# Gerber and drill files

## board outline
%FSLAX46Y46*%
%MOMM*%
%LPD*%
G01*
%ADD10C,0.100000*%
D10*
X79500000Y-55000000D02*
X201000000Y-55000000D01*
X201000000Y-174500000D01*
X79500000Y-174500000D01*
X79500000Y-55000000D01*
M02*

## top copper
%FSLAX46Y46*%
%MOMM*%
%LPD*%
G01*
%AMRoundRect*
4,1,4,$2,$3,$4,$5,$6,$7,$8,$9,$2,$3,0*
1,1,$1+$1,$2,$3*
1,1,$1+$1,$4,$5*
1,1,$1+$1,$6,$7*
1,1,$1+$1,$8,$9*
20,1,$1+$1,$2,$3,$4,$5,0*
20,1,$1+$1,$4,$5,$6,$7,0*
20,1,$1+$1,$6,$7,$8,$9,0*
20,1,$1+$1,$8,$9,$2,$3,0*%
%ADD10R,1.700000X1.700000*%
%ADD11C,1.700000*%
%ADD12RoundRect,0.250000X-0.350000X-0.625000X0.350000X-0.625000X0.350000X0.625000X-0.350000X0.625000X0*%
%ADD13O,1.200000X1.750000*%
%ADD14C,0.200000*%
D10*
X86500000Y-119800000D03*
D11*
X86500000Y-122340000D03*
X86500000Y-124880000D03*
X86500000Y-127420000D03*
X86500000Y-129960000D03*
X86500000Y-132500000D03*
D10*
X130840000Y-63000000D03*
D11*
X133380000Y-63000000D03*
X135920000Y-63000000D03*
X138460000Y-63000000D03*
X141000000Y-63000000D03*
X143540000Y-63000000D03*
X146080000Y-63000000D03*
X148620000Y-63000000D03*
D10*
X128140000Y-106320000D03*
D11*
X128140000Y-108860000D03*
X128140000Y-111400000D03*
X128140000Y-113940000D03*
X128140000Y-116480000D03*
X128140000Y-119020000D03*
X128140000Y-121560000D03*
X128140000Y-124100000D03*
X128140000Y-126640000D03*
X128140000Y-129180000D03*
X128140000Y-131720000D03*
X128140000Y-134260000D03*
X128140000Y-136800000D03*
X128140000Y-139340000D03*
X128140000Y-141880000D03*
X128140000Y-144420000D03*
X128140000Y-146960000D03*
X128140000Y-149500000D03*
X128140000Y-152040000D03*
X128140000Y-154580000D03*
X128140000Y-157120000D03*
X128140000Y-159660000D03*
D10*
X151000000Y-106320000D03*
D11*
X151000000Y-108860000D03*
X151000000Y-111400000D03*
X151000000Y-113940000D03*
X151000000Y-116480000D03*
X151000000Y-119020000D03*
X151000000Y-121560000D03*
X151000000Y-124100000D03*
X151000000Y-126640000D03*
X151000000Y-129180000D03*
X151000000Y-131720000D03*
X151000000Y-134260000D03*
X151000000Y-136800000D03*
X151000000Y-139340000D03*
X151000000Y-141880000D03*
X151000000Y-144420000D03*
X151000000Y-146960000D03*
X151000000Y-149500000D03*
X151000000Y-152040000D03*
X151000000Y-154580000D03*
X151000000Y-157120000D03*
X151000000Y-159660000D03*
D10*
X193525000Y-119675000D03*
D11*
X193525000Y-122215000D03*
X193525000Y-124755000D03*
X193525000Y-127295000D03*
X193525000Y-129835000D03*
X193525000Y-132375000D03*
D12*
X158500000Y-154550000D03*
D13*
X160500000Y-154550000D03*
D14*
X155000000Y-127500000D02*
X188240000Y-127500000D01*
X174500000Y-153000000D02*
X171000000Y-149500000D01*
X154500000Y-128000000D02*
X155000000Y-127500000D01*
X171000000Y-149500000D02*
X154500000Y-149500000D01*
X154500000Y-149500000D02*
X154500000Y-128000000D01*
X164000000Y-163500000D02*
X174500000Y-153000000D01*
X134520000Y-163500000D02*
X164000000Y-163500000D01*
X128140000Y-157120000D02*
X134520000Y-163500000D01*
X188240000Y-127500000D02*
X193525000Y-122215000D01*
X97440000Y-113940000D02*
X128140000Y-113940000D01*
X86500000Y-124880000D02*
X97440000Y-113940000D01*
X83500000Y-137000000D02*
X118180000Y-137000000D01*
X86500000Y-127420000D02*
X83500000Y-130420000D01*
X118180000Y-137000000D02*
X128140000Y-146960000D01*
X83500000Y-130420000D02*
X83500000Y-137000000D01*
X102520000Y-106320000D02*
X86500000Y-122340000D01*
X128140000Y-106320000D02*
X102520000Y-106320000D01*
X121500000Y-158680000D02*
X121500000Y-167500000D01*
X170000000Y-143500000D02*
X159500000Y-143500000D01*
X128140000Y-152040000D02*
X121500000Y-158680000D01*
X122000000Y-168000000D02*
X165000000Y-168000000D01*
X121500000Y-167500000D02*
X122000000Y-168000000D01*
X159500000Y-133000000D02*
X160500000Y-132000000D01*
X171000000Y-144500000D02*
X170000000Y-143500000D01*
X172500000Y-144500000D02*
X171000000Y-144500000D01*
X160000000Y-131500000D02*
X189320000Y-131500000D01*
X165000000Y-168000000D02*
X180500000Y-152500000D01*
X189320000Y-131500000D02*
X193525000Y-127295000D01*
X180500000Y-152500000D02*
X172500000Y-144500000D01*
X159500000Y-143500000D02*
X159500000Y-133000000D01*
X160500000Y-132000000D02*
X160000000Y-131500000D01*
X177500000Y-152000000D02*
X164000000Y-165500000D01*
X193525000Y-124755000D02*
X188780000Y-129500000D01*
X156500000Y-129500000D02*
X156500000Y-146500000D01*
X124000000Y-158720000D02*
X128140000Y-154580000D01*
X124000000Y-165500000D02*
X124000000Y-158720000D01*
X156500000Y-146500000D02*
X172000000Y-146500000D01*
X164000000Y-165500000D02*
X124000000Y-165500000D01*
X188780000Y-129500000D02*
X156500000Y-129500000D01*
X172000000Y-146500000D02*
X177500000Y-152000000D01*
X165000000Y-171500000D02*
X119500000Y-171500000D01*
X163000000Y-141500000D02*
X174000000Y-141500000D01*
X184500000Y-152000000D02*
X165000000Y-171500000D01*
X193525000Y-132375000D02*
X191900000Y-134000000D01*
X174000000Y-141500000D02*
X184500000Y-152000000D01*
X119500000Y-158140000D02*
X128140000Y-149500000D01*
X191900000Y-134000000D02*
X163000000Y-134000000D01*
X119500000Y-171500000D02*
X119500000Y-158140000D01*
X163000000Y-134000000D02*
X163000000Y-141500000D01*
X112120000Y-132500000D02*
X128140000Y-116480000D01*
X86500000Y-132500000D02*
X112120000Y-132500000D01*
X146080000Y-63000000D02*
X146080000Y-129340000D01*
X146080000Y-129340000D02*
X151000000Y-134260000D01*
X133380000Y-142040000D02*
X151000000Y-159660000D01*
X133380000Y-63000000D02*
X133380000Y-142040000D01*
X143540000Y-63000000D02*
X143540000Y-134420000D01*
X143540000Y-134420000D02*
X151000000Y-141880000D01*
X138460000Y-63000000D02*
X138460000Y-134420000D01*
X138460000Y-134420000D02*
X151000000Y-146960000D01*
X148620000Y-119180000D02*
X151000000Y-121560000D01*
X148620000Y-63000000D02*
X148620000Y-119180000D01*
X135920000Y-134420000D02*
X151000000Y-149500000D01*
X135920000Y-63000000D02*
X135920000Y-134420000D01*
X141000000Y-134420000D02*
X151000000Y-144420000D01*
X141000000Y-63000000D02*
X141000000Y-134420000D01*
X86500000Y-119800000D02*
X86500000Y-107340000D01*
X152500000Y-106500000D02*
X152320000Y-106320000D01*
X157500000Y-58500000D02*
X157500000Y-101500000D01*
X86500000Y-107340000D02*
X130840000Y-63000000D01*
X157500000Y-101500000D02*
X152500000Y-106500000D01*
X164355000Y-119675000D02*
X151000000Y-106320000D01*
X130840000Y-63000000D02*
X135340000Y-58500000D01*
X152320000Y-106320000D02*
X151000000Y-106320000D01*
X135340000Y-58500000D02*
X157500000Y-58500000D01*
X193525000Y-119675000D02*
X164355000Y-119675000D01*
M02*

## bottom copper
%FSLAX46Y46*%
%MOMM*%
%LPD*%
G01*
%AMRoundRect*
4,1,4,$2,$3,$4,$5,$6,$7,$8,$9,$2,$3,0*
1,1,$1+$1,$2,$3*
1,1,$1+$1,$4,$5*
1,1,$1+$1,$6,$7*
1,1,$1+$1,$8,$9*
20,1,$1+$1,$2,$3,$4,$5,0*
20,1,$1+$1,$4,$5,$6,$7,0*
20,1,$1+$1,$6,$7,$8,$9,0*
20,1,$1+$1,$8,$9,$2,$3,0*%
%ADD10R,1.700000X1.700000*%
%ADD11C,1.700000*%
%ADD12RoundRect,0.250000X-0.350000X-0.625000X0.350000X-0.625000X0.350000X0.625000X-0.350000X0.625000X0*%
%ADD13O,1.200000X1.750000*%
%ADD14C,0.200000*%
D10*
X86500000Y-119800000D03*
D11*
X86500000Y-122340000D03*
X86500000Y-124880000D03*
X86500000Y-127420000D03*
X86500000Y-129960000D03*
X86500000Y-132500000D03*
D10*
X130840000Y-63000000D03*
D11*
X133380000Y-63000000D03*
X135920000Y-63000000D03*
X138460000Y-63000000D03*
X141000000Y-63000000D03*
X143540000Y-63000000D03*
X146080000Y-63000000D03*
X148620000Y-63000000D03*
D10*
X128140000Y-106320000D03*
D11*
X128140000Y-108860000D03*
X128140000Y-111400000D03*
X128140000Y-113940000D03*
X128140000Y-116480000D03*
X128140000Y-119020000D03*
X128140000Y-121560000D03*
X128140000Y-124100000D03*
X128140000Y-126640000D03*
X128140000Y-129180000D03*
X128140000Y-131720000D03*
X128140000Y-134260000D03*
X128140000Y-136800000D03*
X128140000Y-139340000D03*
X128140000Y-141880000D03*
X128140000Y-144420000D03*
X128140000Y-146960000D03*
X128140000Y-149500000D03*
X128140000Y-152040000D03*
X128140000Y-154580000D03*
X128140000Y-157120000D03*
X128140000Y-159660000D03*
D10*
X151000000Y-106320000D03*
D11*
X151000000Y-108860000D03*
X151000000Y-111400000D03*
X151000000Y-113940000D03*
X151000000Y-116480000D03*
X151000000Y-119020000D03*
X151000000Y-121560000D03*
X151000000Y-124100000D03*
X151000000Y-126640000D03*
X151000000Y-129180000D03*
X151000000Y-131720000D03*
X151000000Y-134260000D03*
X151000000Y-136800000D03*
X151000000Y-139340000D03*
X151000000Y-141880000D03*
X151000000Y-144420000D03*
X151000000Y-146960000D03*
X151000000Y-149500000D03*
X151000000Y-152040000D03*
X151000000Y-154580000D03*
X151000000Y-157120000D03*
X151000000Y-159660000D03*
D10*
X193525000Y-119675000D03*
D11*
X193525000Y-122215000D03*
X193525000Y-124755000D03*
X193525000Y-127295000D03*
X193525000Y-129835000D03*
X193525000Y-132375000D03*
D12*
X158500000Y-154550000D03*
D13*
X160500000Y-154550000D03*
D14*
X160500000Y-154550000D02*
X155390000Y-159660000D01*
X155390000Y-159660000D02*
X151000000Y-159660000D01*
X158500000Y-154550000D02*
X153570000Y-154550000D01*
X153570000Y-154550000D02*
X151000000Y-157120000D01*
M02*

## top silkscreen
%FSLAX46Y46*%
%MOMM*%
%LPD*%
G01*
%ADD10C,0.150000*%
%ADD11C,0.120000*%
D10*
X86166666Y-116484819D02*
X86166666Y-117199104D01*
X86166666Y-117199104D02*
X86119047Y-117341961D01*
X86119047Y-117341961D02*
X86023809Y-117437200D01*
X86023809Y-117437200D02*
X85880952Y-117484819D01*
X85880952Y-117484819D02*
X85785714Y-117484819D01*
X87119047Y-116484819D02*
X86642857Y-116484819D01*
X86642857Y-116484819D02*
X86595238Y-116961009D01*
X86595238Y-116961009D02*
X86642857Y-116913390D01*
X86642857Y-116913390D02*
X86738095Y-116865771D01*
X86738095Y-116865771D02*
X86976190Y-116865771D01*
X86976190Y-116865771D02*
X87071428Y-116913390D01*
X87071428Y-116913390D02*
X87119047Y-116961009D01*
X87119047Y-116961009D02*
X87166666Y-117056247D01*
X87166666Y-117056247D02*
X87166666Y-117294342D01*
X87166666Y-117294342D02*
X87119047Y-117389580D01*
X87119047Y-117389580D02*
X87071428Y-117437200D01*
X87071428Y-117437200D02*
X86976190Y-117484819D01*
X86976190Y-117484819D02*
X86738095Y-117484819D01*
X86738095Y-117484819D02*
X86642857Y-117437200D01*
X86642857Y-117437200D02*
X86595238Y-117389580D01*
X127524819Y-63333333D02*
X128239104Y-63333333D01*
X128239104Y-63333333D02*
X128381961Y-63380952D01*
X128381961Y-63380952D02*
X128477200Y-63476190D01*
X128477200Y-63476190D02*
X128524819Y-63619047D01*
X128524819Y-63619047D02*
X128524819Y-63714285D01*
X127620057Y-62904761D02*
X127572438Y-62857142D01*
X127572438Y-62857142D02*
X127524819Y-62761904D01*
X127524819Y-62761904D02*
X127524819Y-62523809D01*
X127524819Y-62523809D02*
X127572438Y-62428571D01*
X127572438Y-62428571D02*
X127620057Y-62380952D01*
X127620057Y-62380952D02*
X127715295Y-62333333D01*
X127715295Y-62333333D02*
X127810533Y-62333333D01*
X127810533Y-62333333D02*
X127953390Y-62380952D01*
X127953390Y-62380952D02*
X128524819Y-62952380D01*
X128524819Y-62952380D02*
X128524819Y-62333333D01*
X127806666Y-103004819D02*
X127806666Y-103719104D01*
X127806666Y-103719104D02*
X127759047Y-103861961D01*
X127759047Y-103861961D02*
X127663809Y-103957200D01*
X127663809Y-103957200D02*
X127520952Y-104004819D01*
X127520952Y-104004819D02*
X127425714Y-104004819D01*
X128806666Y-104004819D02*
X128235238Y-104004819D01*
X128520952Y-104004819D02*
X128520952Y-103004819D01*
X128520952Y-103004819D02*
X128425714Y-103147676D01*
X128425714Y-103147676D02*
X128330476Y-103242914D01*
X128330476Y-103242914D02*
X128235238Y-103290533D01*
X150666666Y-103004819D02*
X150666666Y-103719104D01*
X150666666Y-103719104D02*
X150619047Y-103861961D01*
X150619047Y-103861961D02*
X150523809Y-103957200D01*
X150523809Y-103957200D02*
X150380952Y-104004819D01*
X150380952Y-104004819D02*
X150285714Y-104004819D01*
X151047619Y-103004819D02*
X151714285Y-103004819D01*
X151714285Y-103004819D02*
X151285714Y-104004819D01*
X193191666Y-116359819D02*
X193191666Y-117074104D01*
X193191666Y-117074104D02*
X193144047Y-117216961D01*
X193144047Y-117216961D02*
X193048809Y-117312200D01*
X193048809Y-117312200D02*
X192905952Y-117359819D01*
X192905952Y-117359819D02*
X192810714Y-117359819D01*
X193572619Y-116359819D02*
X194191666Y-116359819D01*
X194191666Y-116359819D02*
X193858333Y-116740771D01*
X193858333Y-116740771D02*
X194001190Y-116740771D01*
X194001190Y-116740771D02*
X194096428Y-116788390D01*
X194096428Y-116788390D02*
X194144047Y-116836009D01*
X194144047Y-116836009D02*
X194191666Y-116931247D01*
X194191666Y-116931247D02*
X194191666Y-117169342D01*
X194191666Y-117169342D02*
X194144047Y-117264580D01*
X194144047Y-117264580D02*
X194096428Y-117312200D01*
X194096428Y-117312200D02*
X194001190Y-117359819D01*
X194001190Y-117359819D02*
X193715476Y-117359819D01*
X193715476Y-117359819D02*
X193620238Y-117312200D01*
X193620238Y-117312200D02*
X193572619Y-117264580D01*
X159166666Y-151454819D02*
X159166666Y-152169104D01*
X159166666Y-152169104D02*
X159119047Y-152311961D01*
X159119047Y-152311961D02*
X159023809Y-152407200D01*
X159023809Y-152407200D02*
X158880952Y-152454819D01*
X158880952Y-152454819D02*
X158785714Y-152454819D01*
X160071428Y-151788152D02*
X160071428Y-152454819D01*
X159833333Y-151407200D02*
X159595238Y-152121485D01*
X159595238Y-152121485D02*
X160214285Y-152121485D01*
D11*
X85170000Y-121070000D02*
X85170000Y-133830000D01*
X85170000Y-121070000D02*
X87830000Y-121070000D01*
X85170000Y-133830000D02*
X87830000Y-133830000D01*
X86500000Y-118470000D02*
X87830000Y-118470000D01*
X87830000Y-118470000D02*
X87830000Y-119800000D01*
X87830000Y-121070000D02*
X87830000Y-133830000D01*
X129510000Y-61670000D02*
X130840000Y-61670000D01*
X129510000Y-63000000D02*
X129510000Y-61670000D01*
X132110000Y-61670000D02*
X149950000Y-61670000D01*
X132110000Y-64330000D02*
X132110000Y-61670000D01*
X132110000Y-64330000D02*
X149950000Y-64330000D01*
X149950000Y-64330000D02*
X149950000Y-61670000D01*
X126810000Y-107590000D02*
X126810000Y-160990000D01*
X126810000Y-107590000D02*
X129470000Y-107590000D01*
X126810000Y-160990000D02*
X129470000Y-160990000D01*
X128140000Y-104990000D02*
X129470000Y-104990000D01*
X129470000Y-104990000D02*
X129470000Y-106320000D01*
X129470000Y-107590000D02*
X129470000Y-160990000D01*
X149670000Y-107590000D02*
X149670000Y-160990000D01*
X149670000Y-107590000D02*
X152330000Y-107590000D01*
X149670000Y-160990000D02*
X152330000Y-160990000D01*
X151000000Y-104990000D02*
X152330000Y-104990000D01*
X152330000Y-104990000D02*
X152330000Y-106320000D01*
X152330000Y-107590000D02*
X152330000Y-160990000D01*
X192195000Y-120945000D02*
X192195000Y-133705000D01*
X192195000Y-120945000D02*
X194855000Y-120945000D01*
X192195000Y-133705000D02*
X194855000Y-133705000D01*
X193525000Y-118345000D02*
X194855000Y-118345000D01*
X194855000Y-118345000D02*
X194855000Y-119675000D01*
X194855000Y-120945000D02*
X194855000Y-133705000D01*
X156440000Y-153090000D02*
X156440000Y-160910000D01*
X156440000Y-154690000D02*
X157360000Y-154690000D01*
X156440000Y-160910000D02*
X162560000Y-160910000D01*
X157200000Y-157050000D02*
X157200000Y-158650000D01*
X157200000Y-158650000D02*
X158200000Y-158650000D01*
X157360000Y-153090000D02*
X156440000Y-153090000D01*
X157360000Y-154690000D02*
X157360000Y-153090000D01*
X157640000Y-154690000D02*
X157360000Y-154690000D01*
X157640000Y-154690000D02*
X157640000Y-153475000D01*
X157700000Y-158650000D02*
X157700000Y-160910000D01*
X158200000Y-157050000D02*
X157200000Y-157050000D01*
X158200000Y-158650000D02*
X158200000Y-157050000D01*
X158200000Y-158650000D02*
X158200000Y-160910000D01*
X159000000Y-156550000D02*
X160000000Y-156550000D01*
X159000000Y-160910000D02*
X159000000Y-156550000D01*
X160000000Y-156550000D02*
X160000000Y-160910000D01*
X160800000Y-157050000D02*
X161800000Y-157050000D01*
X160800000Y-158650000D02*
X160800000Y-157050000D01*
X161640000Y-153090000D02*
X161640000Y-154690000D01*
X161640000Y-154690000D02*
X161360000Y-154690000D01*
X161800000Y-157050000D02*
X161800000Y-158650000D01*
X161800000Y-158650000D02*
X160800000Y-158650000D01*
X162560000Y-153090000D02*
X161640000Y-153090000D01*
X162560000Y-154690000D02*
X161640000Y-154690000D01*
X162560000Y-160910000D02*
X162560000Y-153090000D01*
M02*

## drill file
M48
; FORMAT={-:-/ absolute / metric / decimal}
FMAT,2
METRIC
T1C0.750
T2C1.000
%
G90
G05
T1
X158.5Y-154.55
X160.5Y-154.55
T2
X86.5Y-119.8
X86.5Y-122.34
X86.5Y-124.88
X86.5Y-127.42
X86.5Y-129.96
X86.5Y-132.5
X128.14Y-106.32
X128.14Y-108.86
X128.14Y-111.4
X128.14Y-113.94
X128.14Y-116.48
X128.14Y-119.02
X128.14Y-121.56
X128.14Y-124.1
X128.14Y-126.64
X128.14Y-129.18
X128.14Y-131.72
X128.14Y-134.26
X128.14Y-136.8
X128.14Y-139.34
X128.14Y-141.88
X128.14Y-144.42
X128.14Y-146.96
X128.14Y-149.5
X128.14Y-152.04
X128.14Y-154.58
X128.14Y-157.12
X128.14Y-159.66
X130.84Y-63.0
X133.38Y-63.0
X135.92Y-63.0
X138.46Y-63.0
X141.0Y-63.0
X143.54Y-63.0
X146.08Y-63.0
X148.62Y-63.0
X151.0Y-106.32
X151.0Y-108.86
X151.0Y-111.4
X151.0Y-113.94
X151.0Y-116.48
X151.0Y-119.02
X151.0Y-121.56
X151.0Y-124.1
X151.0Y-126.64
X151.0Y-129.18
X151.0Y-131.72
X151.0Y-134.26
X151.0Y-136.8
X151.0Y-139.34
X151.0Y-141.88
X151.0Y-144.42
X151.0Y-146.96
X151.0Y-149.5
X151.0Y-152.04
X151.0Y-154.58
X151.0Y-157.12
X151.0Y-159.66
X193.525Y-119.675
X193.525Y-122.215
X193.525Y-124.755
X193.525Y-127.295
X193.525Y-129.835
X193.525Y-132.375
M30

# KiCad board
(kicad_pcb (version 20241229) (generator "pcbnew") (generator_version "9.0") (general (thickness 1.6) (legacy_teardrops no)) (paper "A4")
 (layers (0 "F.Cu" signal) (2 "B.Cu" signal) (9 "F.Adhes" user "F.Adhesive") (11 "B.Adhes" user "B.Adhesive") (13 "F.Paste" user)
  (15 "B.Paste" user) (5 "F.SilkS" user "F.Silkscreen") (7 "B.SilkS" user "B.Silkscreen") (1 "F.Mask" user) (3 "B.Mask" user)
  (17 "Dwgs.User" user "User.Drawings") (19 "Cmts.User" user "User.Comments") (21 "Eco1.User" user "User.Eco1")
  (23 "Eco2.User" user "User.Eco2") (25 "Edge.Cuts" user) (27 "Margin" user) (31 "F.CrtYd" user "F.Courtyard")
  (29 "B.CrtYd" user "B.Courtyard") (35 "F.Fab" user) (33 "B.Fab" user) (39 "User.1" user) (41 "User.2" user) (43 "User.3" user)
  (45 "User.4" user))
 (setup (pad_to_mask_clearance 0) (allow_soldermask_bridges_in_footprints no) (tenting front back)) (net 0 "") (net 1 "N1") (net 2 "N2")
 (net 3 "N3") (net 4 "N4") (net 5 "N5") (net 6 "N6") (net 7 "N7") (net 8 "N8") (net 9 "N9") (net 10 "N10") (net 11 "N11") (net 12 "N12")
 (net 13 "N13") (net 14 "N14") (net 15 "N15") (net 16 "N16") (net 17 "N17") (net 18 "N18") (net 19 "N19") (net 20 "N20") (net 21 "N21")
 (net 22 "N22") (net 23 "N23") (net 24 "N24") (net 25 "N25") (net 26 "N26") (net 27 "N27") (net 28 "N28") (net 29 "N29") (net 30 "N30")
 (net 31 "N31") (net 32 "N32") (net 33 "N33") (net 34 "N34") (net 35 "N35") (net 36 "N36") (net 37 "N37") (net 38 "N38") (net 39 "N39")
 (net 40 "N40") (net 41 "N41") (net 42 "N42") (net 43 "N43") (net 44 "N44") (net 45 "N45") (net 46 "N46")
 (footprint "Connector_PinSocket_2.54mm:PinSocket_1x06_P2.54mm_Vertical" (layer "F.Cu") (at 86.5 119.8)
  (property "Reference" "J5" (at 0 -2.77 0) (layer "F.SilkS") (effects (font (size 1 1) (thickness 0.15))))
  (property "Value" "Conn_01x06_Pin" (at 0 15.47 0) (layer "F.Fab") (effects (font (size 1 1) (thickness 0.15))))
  (fp_line (start -1.33 1.27) (end -1.33 14.03) (stroke (width 0.12) (type solid)) (layer "F.SilkS"))
  (fp_line (start -1.33 1.27) (end 1.33 1.27) (stroke (width 0.12) (type solid)) (layer "F.SilkS"))
  (fp_line (start -1.33 14.03) (end 1.33 14.03) (stroke (width 0.12) (type solid)) (layer "F.SilkS"))
  (fp_line (start 0 -1.33) (end 1.33 -1.33) (stroke (width 0.12) (type solid)) (layer "F.SilkS"))
  (fp_line (start 1.33 -1.33) (end 1.33 0) (stroke (width 0.12) (type solid)) (layer "F.SilkS"))
  (fp_line (start 1.33 1.27) (end 1.33 14.03) (stroke (width 0.12) (type solid)) (layer "F.SilkS"))
  (pad "1" thru_hole rect (at 0 0) (size 1.7 1.7) (drill 1) (layers "*.Cu" "*.Mask") (remove_unused_layers no) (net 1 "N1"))
  (pad "2" thru_hole circle (at 0 2.54) (size 1.7 1.7) (drill 1) (layers "*.Cu" "*.Mask") (remove_unused_layers no) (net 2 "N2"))
  (pad "3" thru_hole circle (at 0 5.08) (size 1.7 1.7) (drill 1) (layers "*.Cu" "*.Mask") (remove_unused_layers no) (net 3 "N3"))
  (pad "4" thru_hole circle (at 0 7.62) (size 1.7 1.7) (drill 1) (layers "*.Cu" "*.Mask") (remove_unused_layers no) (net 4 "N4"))
  (pad "5" thru_hole circle (at 0 10.16) (size 1.7 1.7) (drill 1) (layers "*.Cu" "*.Mask") (remove_unused_layers no) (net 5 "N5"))
  (pad "6" thru_hole circle (at 0 12.7) (size 1.7 1.7) (drill 1) (layers "*.Cu" "*.Mask") (remove_unused_layers no) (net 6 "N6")))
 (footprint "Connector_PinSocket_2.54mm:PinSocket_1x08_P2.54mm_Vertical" (layer "F.Cu") (at 130.84 63 90)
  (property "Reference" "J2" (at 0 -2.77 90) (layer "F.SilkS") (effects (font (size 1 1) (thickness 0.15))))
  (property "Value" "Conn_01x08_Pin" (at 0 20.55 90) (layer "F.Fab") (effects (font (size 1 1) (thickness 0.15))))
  (fp_line (start 1.33 -1.33) (end 1.33 0) (stroke (width 0.12) (type solid)) (layer "F.SilkS"))
  (fp_line (start 0 -1.33) (end 1.33 -1.33) (stroke (width 0.12) (type solid)) (layer "F.SilkS"))
  (fp_line (start 1.33 1.27) (end 1.33 19.11) (stroke (width 0.12) (type solid)) (layer "F.SilkS"))
  (fp_line (start -1.33 1.27) (end 1.33 1.27) (stroke (width 0.12) (type solid)) (layer "F.SilkS"))
  (fp_line (start -1.33 1.27) (end -1.33 19.11) (stroke (width 0.12) (type solid)) (layer "F.SilkS"))
  (fp_line (start -1.33 19.11) (end 1.33 19.11) (stroke (width 0.12) (type solid)) (layer "F.SilkS"))
  (pad "1" thru_hole rect (at 0 0 90) (size 1.7 1.7) (drill 1) (layers "*.Cu" "*.Mask") (remove_unused_layers no) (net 1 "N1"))
  (pad "2" thru_hole circle (at 0 2.54 90) (size 1.7 1.7) (drill 1) (layers "*.Cu" "*.Mask") (remove_unused_layers no) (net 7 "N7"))
  (pad "3" thru_hole circle (at 0 5.08 90) (size 1.7 1.7) (drill 1) (layers "*.Cu" "*.Mask") (remove_unused_layers no) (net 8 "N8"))
  (pad "4" thru_hole circle (at 0 7.62 90) (size 1.7 1.7) (drill 1) (layers "*.Cu" "*.Mask") (remove_unused_layers no) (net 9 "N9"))
  (pad "5" thru_hole circle (at 0 10.16 90) (size 1.7 1.7) (drill 1) (layers "*.Cu" "*.Mask") (remove_unused_layers no) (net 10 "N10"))
  (pad "6" thru_hole circle (at 0 12.7 90) (size 1.7 1.7) (drill 1) (layers "*.Cu" "*.Mask") (remove_unused_layers no) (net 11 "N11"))
  (pad "7" thru_hole circle (at 0 15.24 90) (size 1.7 1.7) (drill 1) (layers "*.Cu" "*.Mask") (remove_unused_layers no) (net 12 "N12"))
  (pad "8" thru_hole circle (at 0 17.78 90) (size 1.7 1.7) (drill 1) (layers "*.Cu" "*.Mask") (remove_unused_layers no) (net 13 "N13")))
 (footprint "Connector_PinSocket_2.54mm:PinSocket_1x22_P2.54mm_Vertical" (layer "F.Cu") (at 128.14 106.32)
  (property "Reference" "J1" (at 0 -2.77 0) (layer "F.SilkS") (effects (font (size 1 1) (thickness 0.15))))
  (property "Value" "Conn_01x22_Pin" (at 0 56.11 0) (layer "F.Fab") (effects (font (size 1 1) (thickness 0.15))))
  (fp_line (start -1.33 1.27) (end -1.33 54.67) (stroke (width 0.12) (type solid)) (layer "F.SilkS"))
  (fp_line (start -1.33 1.27) (end 1.33 1.27) (stroke (width 0.12) (type solid)) (layer "F.SilkS"))
  (fp_line (start -1.33 54.67) (end 1.33 54.67) (stroke (width 0.12) (type solid)) (layer "F.SilkS"))
  (fp_line (start 0 -1.33) (end 1.33 -1.33) (stroke (width 0.12) (type solid)) (layer "F.SilkS"))
  (fp_line (start 1.33 -1.33) (end 1.33 0) (stroke (width 0.12) (type solid)) (layer "F.SilkS"))
  (fp_line (start 1.33 1.27) (end 1.33 54.67) (stroke (width 0.12) (type solid)) (layer "F.SilkS"))
  (pad "1" thru_hole rect (at 0 0) (size 1.7 1.7) (drill 1) (layers "*.Cu" "*.Mask") (remove_unused_layers no) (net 2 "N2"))
  (pad "2" thru_hole circle (at 0 2.54) (size 1.7 1.7) (drill 1) (layers "*.Cu" "*.Mask") (remove_unused_layers no) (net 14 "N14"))
  (pad "3" thru_hole circle (at 0 5.08) (size 1.7 1.7) (drill 1) (layers "*.Cu" "*.Mask") (remove_unused_layers no) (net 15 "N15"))
  (pad "4" thru_hole circle (at 0 7.62) (size 1.7 1.7) (drill 1) (layers "*.Cu" "*.Mask") (remove_unused_layers no) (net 3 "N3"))
  (pad "5" thru_hole circle (at 0 10.16) (size 1.7 1.7) (drill 1) (layers "*.Cu" "*.Mask") (remove_unused_layers no) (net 6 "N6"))
  (pad "6" thru_hole circle (at 0 12.7) (size 1.7 1.7) (drill 1) (layers "*.Cu" "*.Mask") (remove_unused_layers no) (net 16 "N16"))
  (pad "7" thru_hole circle (at 0 15.24) (size 1.7 1.7) (drill 1) (layers "*.Cu" "*.Mask") (remove_unused_layers no) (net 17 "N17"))
  (pad "8" thru_hole circle (at 0 17.78) (size 1.7 1.7) (drill 1) (layers "*.Cu" "*.Mask") (remove_unused_layers no) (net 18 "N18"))
  (pad "9" thru_hole circle (at 0 20.32) (size 1.7 1.7) (drill 1) (layers "*.Cu" "*.Mask") (remove_unused_layers no) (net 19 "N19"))
  (pad "10" thru_hole circle (at 0 22.86) (size 1.7 1.7) (drill 1) (layers "*.Cu" "*.Mask") (remove_unused_layers no) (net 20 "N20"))
  (pad "11" thru_hole circle (at 0 25.4) (size 1.7 1.7) (drill 1) (layers "*.Cu" "*.Mask") (remove_unused_layers no) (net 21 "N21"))
  (pad "12" thru_hole circle (at 0 27.94) (size 1.7 1.7) (drill 1) (layers "*.Cu" "*.Mask") (remove_unused_layers no) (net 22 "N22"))
  (pad "13" thru_hole circle (at 0 30.48) (size 1.7 1.7) (drill 1) (layers "*.Cu" "*.Mask") (remove_unused_layers no) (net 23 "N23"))
  (pad "14" thru_hole circle (at 0 33.02) (size 1.7 1.7) (drill 1) (layers "*.Cu" "*.Mask") (remove_unused_layers no) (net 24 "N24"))
  (pad "15" thru_hole circle (at 0 35.56) (size 1.7 1.7) (drill 1) (layers "*.Cu" "*.Mask") (remove_unused_layers no) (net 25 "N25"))
  (pad "16" thru_hole circle (at 0 38.1) (size 1.7 1.7) (drill 1) (layers "*.Cu" "*.Mask") (remove_unused_layers no) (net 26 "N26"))
  (pad "17" thru_hole circle (at 0 40.64) (size 1.7 1.7) (drill 1) (layers "*.Cu" "*.Mask") (remove_unused_layers no) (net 4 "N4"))
  (pad "18" thru_hole circle (at 0 43.18) (size 1.7 1.7) (drill 1) (layers "*.Cu" "*.Mask") (remove_unused_layers no) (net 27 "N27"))
  (pad "19" thru_hole circle (at 0 45.72) (size 1.7 1.7) (drill 1) (layers "*.Cu" "*.Mask") (remove_unused_layers no) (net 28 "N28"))
  (pad "20" thru_hole circle (at 0 48.26) (size 1.7 1.7) (drill 1) (layers "*.Cu" "*.Mask") (remove_unused_layers no) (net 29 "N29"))
  (pad "21" thru_hole circle (at 0 50.8) (size 1.7 1.7) (drill 1) (layers "*.Cu" "*.Mask") (remove_unused_layers no) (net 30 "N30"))
  (pad "22" thru_hole circle (at 0 53.34) (size 1.7 1.7) (drill 1) (layers "*.Cu" "*.Mask") (remove_unused_layers no) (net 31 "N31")))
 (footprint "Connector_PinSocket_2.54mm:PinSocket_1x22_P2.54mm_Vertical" (layer "F.Cu") (at 151 106.32)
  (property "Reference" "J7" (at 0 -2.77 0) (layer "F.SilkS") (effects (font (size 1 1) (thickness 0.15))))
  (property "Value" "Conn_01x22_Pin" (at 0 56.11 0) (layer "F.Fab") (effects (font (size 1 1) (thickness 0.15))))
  (fp_line (start -1.33 1.27) (end -1.33 54.67) (stroke (width 0.12) (type solid)) (layer "F.SilkS"))
  (fp_line (start -1.33 1.27) (end 1.33 1.27) (stroke (width 0.12) (type solid)) (layer "F.SilkS"))
  (fp_line (start -1.33 54.67) (end 1.33 54.67) (stroke (width 0.12) (type solid)) (layer "F.SilkS"))
  (fp_line (start 0 -1.33) (end 1.33 -1.33) (stroke (width 0.12) (type solid)) (layer "F.SilkS"))
  (fp_line (start 1.33 -1.33) (end 1.33 0) (stroke (width 0.12) (type solid)) (layer "F.SilkS"))
  (fp_line (start 1.33 1.27) (end 1.33 54.67) (stroke (width 0.12) (type solid)) (layer "F.SilkS"))
  (pad "1" thru_hole rect (at 0 0) (size 1.7 1.7) (drill 1) (layers "*.Cu" "*.Mask") (remove_unused_layers no) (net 1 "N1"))
  (pad "2" thru_hole circle (at 0 2.54) (size 1.7 1.7) (drill 1) (layers "*.Cu" "*.Mask") (remove_unused_layers no) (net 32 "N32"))
  (pad "3" thru_hole circle (at 0 5.08) (size 1.7 1.7) (drill 1) (layers "*.Cu" "*.Mask") (remove_unused_layers no) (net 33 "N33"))
  (pad "4" thru_hole circle (at 0 7.62) (size 1.7 1.7) (drill 1) (layers "*.Cu" "*.Mask") (remove_unused_layers no) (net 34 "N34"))
  (pad "5" thru_hole circle (at 0 10.16) (size 1.7 1.7) (drill 1) (layers "*.Cu" "*.Mask") (remove_unused_layers no) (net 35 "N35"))
  (pad "6" thru_hole circle (at 0 12.7) (size 1.7 1.7) (drill 1) (layers "*.Cu" "*.Mask") (remove_unused_layers no) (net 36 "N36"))
  (pad "7" thru_hole circle (at 0 15.24) (size 1.7 1.7) (drill 1) (layers "*.Cu" "*.Mask") (remove_unused_layers no) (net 13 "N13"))
  (pad "8" thru_hole circle (at 0 17.78) (size 1.7 1.7) (drill 1) (layers "*.Cu" "*.Mask") (remove_unused_layers no) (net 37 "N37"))
  (pad "9" thru_hole circle (at 0 20.32) (size 1.7 1.7) (drill 1) (layers "*.Cu" "*.Mask") (remove_unused_layers no) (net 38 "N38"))
  (pad "10" thru_hole circle (at 0 22.86) (size 1.7 1.7) (drill 1) (layers "*.Cu" "*.Mask") (remove_unused_layers no) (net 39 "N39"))
  (pad "11" thru_hole circle (at 0 25.4) (size 1.7 1.7) (drill 1) (layers "*.Cu" "*.Mask") (remove_unused_layers no) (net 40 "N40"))
  (pad "12" thru_hole circle (at 0 27.94) (size 1.7 1.7) (drill 1) (layers "*.Cu" "*.Mask") (remove_unused_layers no) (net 12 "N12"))
  (pad "13" thru_hole circle (at 0 30.48) (size 1.7 1.7) (drill 1) (layers "*.Cu" "*.Mask") (remove_unused_layers no) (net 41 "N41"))
  (pad "14" thru_hole circle (at 0 33.02) (size 1.7 1.7) (drill 1) (layers "*.Cu" "*.Mask") (remove_unused_layers no) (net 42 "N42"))
  (pad "15" thru_hole circle (at 0 35.56) (size 1.7 1.7) (drill 1) (layers "*.Cu" "*.Mask") (remove_unused_layers no) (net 11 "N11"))
  (pad "16" thru_hole circle (at 0 38.1) (size 1.7 1.7) (drill 1) (layers "*.Cu" "*.Mask") (remove_unused_layers no) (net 10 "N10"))
  (pad "17" thru_hole circle (at 0 40.64) (size 1.7 1.7) (drill 1) (layers "*.Cu" "*.Mask") (remove_unused_layers no) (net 9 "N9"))
  (pad "18" thru_hole circle (at 0 43.18) (size 1.7 1.7) (drill 1) (layers "*.Cu" "*.Mask") (remove_unused_layers no) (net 8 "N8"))
  (pad "19" thru_hole circle (at 0 45.72) (size 1.7 1.7) (drill 1) (layers "*.Cu" "*.Mask") (remove_unused_layers no) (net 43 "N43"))
  (pad "20" thru_hole circle (at 0 48.26) (size 1.7 1.7) (drill 1) (layers "*.Cu" "*.Mask") (remove_unused_layers no) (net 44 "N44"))
  (pad "21" thru_hole circle (at 0 50.8) (size 1.7 1.7) (drill 1) (layers "*.Cu" "*.Mask") (remove_unused_layers no) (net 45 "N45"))
  (pad "22" thru_hole circle (at 0 53.34) (size 1.7 1.7) (drill 1) (layers "*.Cu" "*.Mask") (remove_unused_layers no) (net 7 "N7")))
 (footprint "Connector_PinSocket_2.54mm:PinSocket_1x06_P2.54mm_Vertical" (layer "F.Cu") (at 193.525 119.675)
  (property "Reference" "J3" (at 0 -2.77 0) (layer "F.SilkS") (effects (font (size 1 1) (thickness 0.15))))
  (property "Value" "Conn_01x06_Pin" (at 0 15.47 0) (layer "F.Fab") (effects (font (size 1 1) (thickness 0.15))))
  (fp_line (start -1.33 1.27) (end -1.33 14.03) (stroke (width 0.12) (type solid)) (layer "F.SilkS"))
  (fp_line (start -1.33 1.27) (end 1.33 1.27) (stroke (width 0.12) (type solid)) (layer "F.SilkS"))
  (fp_line (start -1.33 14.03) (end 1.33 14.03) (stroke (width 0.12) (type solid)) (layer "F.SilkS"))
  (fp_line (start 0 -1.33) (end 1.33 -1.33) (stroke (width 0.12) (type solid)) (layer "F.SilkS"))
  (fp_line (start 1.33 -1.33) (end 1.33 0) (stroke (width 0.12) (type solid)) (layer "F.SilkS"))
  (fp_line (start 1.33 1.27) (end 1.33 14.03) (stroke (width 0.12) (type solid)) (layer "F.SilkS"))
  (pad "1" thru_hole rect (at 0 0) (size 1.7 1.7) (drill 1) (layers "*.Cu" "*.Mask") (remove_unused_layers no) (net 1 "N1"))
  (pad "2" thru_hole circle (at 0 2.54) (size 1.7 1.7) (drill 1) (layers "*.Cu" "*.Mask") (remove_unused_layers no) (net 30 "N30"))
  (pad "3" thru_hole circle (at 0 5.08) (size 1.7 1.7) (drill 1) (layers "*.Cu" "*.Mask") (remove_unused_layers no) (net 29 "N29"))
  (pad "4" thru_hole circle (at 0 7.62) (size 1.7 1.7) (drill 1) (layers "*.Cu" "*.Mask") (remove_unused_layers no) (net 28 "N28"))
  (pad "5" thru_hole circle (at 0 10.16) (size 1.7 1.7) (drill 1) (layers "*.Cu" "*.Mask") (remove_unused_layers no) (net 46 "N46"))
  (pad "6" thru_hole circle (at 0 12.7) (size 1.7 1.7) (drill 1) (layers "*.Cu" "*.Mask") (remove_unused_layers no) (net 27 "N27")))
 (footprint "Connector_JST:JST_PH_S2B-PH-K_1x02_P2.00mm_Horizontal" (layer "F.Cu") (at 158.5 154.55)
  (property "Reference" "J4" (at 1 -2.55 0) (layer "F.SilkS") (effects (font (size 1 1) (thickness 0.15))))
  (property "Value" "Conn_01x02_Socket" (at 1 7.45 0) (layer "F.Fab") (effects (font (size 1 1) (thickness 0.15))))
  (fp_line (start -2.06 -1.46) (end -2.06 6.36) (stroke (width 0.12) (type solid)) (layer "F.SilkS"))
  (fp_line (start -2.06 0.14) (end -1.14 0.14) (stroke (width 0.12) (type solid)) (layer "F.SilkS"))
  (fp_line (start -2.06 6.36) (end 4.06 6.36) (stroke (width 0.12) (type solid)) (layer "F.SilkS"))
  (fp_line (start -1.3 2.5) (end -1.3 4.1) (stroke (width 0.12) (type solid)) (layer "F.SilkS"))
  (fp_line (start -1.3 4.1) (end -0.3 4.1) (stroke (width 0.12) (type solid)) (layer "F.SilkS"))
  (fp_line (start -1.14 -1.46) (end -2.06 -1.46) (stroke (width 0.12) (type solid)) (layer "F.SilkS"))
  (fp_line (start -1.14 0.14) (end -1.14 -1.46) (stroke (width 0.12) (type solid)) (layer "F.SilkS"))
  (fp_line (start -0.86 0.14) (end -1.14 0.14) (stroke (width 0.12) (type solid)) (layer "F.SilkS"))
  (fp_line (start -0.86 0.14) (end -0.86 -1.075) (stroke (width 0.12) (type solid)) (layer "F.SilkS"))
  (fp_line (start -0.8 4.1) (end -0.8 6.36) (stroke (width 0.12) (type solid)) (layer "F.SilkS"))
  (fp_line (start -0.3 2.5) (end -1.3 2.5) (stroke (width 0.12) (type solid)) (layer "F.SilkS"))
  (fp_line (start -0.3 4.1) (end -0.3 2.5) (stroke (width 0.12) (type solid)) (layer "F.SilkS"))
  (fp_line (start -0.3 4.1) (end -0.3 6.36) (stroke (width 0.12) (type solid)) (layer "F.SilkS"))
  (fp_line (start 0.5 2) (end 1.5 2) (stroke (width 0.12) (type solid)) (layer "F.SilkS"))
  (fp_line (start 0.5 6.36) (end 0.5 2) (stroke (width 0.12) (type solid)) (layer "F.SilkS"))
  (fp_line (start 1.5 2) (end 1.5 6.36) (stroke (width 0.12) (type solid)) (layer "F.SilkS"))
  (fp_line (start 2.3 2.5) (end 3.3 2.5) (stroke (width 0.12) (type solid)) (layer "F.SilkS"))
  (fp_line (start 2.3 4.1) (end 2.3 2.5) (stroke (width 0.12) (type solid)) (layer "F.SilkS"))
  (fp_line (start 3.14 -1.46) (end 3.14 0.14) (stroke (width 0.12) (type solid)) (layer "F.SilkS"))
  (fp_line (start 3.14 0.14) (end 2.86 0.14) (stroke (width 0.12) (type solid)) (layer "F.SilkS"))
  (fp_line (start 3.3 2.5) (end 3.3 4.1) (stroke (width 0.12) (type solid)) (layer "F.SilkS"))
  (fp_line (start 3.3 4.1) (end 2.3 4.1) (stroke (width 0.12) (type solid)) (layer "F.SilkS"))
  (fp_line (start 4.06 -1.46) (end 3.14 -1.46) (stroke (width 0.12) (type solid)) (layer "F.SilkS"))
  (fp_line (start 4.06 0.14) (end 3.14 0.14) (stroke (width 0.12) (type solid)) (layer "F.SilkS"))
  (fp_line (start 4.06 6.36) (end 4.06 -1.46) (stroke (width 0.12) (type solid)) (layer "F.SilkS"))
  (pad "1" thru_hole roundrect (at 0 0) (size 1.2 1.75) (drill 0.75) (layers "*.Cu" "*.Mask") (remove_unused_layers no)
   (roundrect_rratio 0.208333) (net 45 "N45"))
  (pad "2" thru_hole oval (at 2 0) (size 1.2 1.75) (drill 0.75) (layers "*.Cu" "*.Mask") (remove_unused_layers no) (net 7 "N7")))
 (gr_rect (start 79.5 55) (end 201 174.5) (stroke (width 0.1) (type default)) (fill no) (layer "Edge.Cuts"))
 (segment (start 155 127.5) (end 188.24 127.5) (width 0.2) (layer "F.Cu") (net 30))
 (segment (start 174.5 153) (end 171 149.5) (width 0.2) (layer "F.Cu") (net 30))
 (segment (start 154.5 128) (end 155 127.5) (width 0.2) (layer "F.Cu") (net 30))
 (segment (start 171 149.5) (end 154.5 149.5) (width 0.2) (layer "F.Cu") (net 30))
 (segment (start 154.5 149.5) (end 154.5 128) (width 0.2) (layer "F.Cu") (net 30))
 (segment (start 164 163.5) (end 174.5 153) (width 0.2) (layer "F.Cu") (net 30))
 (segment (start 134.52 163.5) (end 164 163.5) (width 0.2) (layer "F.Cu") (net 30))
 (segment (start 128.14 157.12) (end 134.52 163.5) (width 0.2) (layer "F.Cu") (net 30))
 (segment (start 188.24 127.5) (end 193.525 122.215) (width 0.2) (layer "F.Cu") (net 30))
 (segment (start 97.44 113.94) (end 128.14 113.94) (width 0.2) (layer "F.Cu") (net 3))
 (segment (start 86.5 124.88) (end 97.44 113.94) (width 0.2) (layer "F.Cu") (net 3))
 (segment (start 83.5 137) (end 118.18 137) (width 0.2) (layer "F.Cu") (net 4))
 (segment (start 86.5 127.42) (end 83.5 130.42) (width 0.2) (layer "F.Cu") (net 4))
 (segment (start 118.18 137) (end 128.14 146.96) (width 0.2) (layer "F.Cu") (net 4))
 (segment (start 83.5 130.42) (end 83.5 137) (width 0.2) (layer "F.Cu") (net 4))
 (segment (start 102.52 106.32) (end 86.5 122.34) (width 0.2) (layer "F.Cu") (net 2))
 (segment (start 128.14 106.32) (end 102.52 106.32) (width 0.2) (layer "F.Cu") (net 2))
 (segment (start 121.5 158.68) (end 121.5 167.5) (width 0.2) (layer "F.Cu") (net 28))
 (segment (start 170 143.5) (end 159.5 143.5) (width 0.2) (layer "F.Cu") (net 28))
 (segment (start 128.14 152.04) (end 121.5 158.68) (width 0.2) (layer "F.Cu") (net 28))
 (segment (start 122 168) (end 165 168) (width 0.2) (layer "F.Cu") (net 28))
 (segment (start 121.5 167.5) (end 122 168) (width 0.2) (layer "F.Cu") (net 28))
 (segment (start 159.5 133) (end 160.5 132) (width 0.2) (layer "F.Cu") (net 28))
 (segment (start 171 144.5) (end 170 143.5) (width 0.2) (layer "F.Cu") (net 28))
 (segment (start 172.5 144.5) (end 171 144.5) (width 0.2) (layer "F.Cu") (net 28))
 (segment (start 160 131.5) (end 189.32 131.5) (width 0.2) (layer "F.Cu") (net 28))
 (segment (start 165 168) (end 180.5 152.5) (width 0.2) (layer "F.Cu") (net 28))
 (segment (start 189.32 131.5) (end 193.525 127.295) (width 0.2) (layer "F.Cu") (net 28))
 (segment (start 180.5 152.5) (end 172.5 144.5) (width 0.2) (layer "F.Cu") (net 28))
 (segment (start 159.5 143.5) (end 159.5 133) (width 0.2) (layer "F.Cu") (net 28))
 (segment (start 160.5 132) (end 160 131.5) (width 0.2) (layer "F.Cu") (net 28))
 (segment (start 177.5 152) (end 164 165.5) (width 0.2) (layer "F.Cu") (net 29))
 (segment (start 193.525 124.755) (end 188.78 129.5) (width 0.2) (layer "F.Cu") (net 29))
 (segment (start 156.5 129.5) (end 156.5 146.5) (width 0.2) (layer "F.Cu") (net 29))
 (segment (start 124 158.72) (end 128.14 154.58) (width 0.2) (layer "F.Cu") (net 29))
 (segment (start 124 165.5) (end 124 158.72) (width 0.2) (layer "F.Cu") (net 29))
 (segment (start 156.5 146.5) (end 172 146.5) (width 0.2) (layer "F.Cu") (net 29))
 (segment (start 164 165.5) (end 124 165.5) (width 0.2) (layer "F.Cu") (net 29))
 (segment (start 188.78 129.5) (end 156.5 129.5) (width 0.2) (layer "F.Cu") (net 29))
 (segment (start 172 146.5) (end 177.5 152) (width 0.2) (layer "F.Cu") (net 29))
 (segment (start 165 171.5) (end 119.5 171.5) (width 0.2) (layer "F.Cu") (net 27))
 (segment (start 163 141.5) (end 174 141.5) (width 0.2) (layer "F.Cu") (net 27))
 (segment (start 184.5 152) (end 165 171.5) (width 0.2) (layer "F.Cu") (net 27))
 (segment (start 193.525 132.375) (end 191.9 134) (width 0.2) (layer "F.Cu") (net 27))
 (segment (start 174 141.5) (end 184.5 152) (width 0.2) (layer "F.Cu") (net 27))
 (segment (start 119.5 158.14) (end 128.14 149.5) (width 0.2) (layer "F.Cu") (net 27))
 (segment (start 191.9 134) (end 163 134) (width 0.2) (layer "F.Cu") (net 27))
 (segment (start 119.5 171.5) (end 119.5 158.14) (width 0.2) (layer "F.Cu") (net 27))
 (segment (start 163 134) (end 163 141.5) (width 0.2) (layer "F.Cu") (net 27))
 (segment (start 112.12 132.5) (end 128.14 116.48) (width 0.2) (layer "F.Cu") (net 6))
 (segment (start 86.5 132.5) (end 112.12 132.5) (width 0.2) (layer "F.Cu") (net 6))
 (segment (start 146.08 63) (end 146.08 129.34) (width 0.2) (layer "F.Cu") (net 12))
 (segment (start 146.08 129.34) (end 151 134.26) (width 0.2) (layer "F.Cu") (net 12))
 (segment (start 133.38 142.04) (end 151 159.66) (width 0.2) (layer "F.Cu") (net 7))
 (segment (start 133.38 63) (end 133.38 142.04) (width 0.2) (layer "F.Cu") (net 7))
 (segment (start 160.5 154.55) (end 155.39 159.66) (width 0.2) (layer "B.Cu") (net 7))
 (segment (start 155.39 159.66) (end 151 159.66) (width 0.2) (layer "B.Cu") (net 7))
 (segment (start 143.54 63) (end 143.54 134.42) (width 0.2) (layer "F.Cu") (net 11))
 (segment (start 143.54 134.42) (end 151 141.88) (width 0.2) (layer "F.Cu") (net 11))
 (segment (start 138.46 63) (end 138.46 134.42) (width 0.2) (layer "F.Cu") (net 9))
 (segment (start 138.46 134.42) (end 151 146.96) (width 0.2) (layer "F.Cu") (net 9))
 (segment (start 148.62 119.18) (end 151 121.56) (width 0.2) (layer "F.Cu") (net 13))
 (segment (start 148.62 63) (end 148.62 119.18) (width 0.2) (layer "F.Cu") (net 13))
 (segment (start 135.92 134.42) (end 151 149.5) (width 0.2) (layer "F.Cu") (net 8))
 (segment (start 135.92 63) (end 135.92 134.42) (width 0.2) (layer "F.Cu") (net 8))
 (segment (start 141 134.42) (end 151 144.42) (width 0.2) (layer "F.Cu") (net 10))
 (segment (start 141 63) (end 141 134.42) (width 0.2) (layer "F.Cu") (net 10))
 (segment (start 86.5 119.8) (end 86.5 107.34) (width 0.2) (layer "F.Cu") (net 1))
 (segment (start 152.5 106.5) (end 152.32 106.32) (width 0.2) (layer "F.Cu") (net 1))
 (segment (start 157.5 58.5) (end 157.5 101.5) (width 0.2) (layer "F.Cu") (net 1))
 (segment (start 86.5 107.34) (end 130.84 63) (width 0.2) (layer "F.Cu") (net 1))
 (segment (start 157.5 101.5) (end 152.5 106.5) (width 0.2) (layer "F.Cu") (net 1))
 (segment (start 164.355 119.675) (end 151 106.32) (width 0.2) (layer "F.Cu") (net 1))
 (segment (start 130.84 63) (end 135.34 58.5) (width 0.2) (layer "F.Cu") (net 1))
 (segment (start 152.32 106.32) (end 151 106.32) (width 0.2) (layer "F.Cu") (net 1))
 (segment (start 135.34 58.5) (end 157.5 58.5) (width 0.2) (layer "F.Cu") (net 1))
 (segment (start 193.525 119.675) (end 164.355 119.675) (width 0.2) (layer "F.Cu") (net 1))
 (segment (start 158.5 154.55) (end 153.57 154.55) (width 0.2) (layer "B.Cu") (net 45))
 (segment (start 153.57 154.55) (end 151 157.12) (width 0.2) (layer "B.Cu") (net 45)))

